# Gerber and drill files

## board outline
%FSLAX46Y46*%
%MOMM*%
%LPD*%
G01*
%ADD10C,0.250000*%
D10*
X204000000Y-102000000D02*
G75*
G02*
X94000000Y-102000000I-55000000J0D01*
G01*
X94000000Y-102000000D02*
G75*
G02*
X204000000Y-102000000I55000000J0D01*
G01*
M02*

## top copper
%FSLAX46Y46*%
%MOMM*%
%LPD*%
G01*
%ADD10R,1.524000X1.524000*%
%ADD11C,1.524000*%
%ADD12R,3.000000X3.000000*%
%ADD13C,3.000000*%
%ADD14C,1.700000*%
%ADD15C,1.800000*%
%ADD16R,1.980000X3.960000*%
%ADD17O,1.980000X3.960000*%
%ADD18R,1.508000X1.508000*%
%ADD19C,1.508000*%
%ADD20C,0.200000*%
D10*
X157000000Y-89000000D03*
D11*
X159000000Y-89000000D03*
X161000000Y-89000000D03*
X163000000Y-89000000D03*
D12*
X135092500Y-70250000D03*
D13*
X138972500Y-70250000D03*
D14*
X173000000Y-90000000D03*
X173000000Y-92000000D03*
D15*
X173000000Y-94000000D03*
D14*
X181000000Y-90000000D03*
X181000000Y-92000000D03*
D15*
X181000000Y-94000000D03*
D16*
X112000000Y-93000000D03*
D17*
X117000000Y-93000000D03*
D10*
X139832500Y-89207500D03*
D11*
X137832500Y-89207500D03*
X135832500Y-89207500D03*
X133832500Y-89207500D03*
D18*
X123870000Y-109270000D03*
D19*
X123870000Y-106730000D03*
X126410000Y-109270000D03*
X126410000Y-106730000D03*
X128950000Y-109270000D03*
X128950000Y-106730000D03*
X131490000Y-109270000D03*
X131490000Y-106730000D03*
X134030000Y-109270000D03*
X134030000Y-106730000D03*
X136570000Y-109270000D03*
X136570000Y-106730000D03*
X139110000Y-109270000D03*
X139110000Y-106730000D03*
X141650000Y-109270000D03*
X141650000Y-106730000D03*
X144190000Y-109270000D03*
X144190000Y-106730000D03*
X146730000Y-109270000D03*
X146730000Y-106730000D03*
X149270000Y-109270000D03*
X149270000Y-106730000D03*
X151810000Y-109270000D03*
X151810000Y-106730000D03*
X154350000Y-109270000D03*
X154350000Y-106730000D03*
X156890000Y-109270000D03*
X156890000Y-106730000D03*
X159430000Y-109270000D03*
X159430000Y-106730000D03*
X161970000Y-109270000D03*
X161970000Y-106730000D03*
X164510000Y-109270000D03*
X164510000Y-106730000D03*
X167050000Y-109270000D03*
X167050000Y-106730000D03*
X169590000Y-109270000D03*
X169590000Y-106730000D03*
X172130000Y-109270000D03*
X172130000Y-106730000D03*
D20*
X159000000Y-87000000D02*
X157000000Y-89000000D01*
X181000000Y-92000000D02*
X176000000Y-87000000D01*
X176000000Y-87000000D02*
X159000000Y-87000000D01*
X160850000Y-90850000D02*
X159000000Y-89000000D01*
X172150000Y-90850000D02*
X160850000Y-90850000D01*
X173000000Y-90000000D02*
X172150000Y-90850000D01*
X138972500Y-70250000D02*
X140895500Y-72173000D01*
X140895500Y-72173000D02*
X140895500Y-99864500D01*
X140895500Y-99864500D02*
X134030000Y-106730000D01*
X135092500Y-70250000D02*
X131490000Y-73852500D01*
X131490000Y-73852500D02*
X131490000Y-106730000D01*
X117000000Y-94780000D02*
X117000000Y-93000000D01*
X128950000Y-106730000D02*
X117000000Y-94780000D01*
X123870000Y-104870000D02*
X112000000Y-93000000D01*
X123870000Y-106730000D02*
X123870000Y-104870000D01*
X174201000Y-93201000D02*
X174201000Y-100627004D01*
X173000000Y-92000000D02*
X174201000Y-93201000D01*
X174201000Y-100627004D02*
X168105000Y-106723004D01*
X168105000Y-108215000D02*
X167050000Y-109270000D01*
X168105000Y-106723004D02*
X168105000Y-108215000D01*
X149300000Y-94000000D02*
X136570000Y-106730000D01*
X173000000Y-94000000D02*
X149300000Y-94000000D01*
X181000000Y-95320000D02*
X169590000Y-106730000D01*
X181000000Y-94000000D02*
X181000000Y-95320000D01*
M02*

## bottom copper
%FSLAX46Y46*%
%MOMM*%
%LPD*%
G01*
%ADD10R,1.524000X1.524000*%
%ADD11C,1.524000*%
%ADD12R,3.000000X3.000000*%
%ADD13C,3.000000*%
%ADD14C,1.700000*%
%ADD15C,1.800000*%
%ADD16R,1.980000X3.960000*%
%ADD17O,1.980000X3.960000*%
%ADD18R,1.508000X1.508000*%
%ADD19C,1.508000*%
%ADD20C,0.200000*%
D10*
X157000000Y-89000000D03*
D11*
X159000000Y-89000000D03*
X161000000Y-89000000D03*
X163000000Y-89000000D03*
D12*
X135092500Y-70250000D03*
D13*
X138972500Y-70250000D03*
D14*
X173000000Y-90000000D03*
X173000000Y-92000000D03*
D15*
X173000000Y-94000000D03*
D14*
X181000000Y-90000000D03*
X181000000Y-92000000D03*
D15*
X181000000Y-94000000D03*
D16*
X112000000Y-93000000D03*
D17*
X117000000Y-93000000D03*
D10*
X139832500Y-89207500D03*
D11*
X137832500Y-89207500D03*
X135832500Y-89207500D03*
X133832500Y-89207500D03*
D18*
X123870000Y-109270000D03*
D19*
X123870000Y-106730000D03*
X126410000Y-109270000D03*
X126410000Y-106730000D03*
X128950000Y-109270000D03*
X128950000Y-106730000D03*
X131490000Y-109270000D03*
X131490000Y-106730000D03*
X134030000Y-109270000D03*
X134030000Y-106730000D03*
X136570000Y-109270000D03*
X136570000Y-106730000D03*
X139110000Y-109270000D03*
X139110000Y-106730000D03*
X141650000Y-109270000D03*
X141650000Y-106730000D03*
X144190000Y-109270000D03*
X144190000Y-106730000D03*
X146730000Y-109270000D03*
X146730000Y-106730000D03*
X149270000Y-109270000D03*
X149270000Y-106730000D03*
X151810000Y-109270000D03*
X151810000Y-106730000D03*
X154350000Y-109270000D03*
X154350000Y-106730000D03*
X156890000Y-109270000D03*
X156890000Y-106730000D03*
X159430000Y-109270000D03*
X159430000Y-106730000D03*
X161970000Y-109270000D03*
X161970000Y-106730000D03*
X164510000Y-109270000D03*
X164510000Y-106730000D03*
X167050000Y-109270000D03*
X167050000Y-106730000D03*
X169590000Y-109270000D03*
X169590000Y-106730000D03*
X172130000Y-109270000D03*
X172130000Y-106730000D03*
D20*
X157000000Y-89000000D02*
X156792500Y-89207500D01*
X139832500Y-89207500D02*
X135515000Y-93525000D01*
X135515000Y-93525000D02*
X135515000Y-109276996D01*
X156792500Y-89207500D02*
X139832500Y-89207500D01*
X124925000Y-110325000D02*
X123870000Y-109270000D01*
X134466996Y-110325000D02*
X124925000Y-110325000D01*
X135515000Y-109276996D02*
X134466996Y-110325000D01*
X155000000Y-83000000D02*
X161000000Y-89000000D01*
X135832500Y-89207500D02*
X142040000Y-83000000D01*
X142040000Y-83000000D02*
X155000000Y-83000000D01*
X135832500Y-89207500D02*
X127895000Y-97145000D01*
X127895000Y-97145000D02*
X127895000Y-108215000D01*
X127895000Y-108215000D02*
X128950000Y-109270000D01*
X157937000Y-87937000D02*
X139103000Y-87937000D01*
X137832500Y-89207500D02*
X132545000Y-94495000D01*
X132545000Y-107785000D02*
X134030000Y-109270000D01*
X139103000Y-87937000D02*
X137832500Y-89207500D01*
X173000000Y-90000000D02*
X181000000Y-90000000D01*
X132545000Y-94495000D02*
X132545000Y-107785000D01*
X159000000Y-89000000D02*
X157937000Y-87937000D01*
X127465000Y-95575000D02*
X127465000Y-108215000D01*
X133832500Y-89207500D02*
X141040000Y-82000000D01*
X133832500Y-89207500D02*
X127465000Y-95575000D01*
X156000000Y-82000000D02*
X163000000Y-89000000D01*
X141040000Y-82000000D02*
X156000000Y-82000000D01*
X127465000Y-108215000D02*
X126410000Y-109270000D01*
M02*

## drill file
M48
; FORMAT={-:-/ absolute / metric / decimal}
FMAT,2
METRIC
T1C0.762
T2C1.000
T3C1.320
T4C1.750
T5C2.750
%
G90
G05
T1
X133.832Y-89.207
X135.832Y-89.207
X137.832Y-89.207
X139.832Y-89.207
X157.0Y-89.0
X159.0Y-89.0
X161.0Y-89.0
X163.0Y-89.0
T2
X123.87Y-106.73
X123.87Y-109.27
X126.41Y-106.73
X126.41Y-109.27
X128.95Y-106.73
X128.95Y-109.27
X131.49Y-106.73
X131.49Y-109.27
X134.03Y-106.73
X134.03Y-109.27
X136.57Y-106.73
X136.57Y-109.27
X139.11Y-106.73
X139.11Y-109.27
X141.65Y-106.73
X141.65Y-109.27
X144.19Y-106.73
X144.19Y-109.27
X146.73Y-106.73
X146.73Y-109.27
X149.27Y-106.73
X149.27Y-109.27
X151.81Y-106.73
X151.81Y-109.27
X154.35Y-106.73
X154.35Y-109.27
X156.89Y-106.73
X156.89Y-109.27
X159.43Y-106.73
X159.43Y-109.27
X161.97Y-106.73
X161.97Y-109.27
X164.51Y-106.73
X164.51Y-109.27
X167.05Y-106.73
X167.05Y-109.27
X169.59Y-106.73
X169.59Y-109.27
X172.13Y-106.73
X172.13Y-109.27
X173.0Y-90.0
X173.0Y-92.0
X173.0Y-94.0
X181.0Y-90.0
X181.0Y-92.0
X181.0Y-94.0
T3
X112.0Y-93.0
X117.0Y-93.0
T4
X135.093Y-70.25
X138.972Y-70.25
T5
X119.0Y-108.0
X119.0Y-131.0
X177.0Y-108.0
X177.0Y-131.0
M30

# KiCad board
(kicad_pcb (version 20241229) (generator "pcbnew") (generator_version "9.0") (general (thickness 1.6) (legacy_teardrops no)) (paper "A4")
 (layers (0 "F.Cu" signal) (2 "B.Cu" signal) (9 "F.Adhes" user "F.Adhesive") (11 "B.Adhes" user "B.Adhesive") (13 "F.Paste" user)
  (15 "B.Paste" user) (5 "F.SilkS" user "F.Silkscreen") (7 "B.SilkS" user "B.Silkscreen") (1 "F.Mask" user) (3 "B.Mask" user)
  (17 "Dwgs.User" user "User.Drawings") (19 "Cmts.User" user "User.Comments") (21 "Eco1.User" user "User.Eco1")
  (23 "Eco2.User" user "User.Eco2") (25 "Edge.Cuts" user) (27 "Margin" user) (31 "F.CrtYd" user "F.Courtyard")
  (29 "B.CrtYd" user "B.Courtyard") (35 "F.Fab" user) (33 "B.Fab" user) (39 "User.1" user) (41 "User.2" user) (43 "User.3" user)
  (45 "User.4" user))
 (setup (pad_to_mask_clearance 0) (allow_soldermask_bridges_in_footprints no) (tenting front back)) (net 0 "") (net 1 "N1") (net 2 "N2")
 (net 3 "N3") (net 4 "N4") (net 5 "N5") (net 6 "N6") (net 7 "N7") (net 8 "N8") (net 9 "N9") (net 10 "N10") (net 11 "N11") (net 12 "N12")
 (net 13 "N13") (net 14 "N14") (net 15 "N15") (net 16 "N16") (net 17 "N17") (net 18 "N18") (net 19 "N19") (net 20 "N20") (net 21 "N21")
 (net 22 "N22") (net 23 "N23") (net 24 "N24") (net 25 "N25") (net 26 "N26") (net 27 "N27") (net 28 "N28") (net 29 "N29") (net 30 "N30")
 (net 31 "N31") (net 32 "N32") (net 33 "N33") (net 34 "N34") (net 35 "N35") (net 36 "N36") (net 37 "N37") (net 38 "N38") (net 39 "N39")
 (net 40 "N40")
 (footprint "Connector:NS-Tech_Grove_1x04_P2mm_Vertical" (layer "F.Cu") (at 157 89 90)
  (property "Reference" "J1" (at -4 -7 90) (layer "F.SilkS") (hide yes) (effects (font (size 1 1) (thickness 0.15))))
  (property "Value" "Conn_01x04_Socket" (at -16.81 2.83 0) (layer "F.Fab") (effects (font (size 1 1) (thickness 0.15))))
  (pad "1" thru_hole rect (at 0 0 90) (size 1.524 1.524) (drill 0.762) (layers "*.Cu" "*.Mask") (remove_unused_layers no) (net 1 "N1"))
  (pad "2" thru_hole circle (at 0 2 90) (size 1.524 1.524) (drill 0.762) (layers "*.Cu" "*.Mask") (remove_unused_layers no) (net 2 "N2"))
  (pad "3" thru_hole circle (at 0 4 90) (size 1.524 1.524) (drill 0.762) (layers "*.Cu" "*.Mask") (remove_unused_layers no) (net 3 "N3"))
  (pad "4" thru_hole circle (at 0 6 90) (size 1.524 1.524) (drill 0.762) (layers "*.Cu" "*.Mask") (remove_unused_layers no) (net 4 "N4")))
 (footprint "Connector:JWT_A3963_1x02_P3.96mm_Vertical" (layer "F.Cu") (at 135.0925 70.25)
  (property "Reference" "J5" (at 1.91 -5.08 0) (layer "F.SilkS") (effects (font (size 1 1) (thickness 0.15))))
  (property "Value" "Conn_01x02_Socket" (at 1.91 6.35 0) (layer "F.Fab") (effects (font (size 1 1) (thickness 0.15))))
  (pad "1" thru_hole rect (at 0 0) (size 3 3) (drill 1.75) (layers "*.Cu" "*.Mask") (remove_unused_layers no) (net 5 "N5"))
  (pad "2" thru_hole circle (at 3.88 0) (size 3 3) (drill 1.75) (layers "*.Cu" "*.Mask") (remove_unused_layers no) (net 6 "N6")))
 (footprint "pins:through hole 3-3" (layer "F.Cu") (at 162 77)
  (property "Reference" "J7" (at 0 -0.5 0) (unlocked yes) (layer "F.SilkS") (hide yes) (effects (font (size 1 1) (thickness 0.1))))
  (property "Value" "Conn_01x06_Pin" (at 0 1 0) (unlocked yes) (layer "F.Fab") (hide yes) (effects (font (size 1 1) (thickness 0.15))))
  (pad "1" thru_hole circle (at 11 13) (size 1.7 1.7) (drill 1) (layers "*.Cu" "*.Mask") (remove_unused_layers no) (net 2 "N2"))
  (pad "2" thru_hole circle (at 11 15) (size 1.7 1.7) (drill 1) (layers "*.Cu" "*.Mask" "B.SilkS") (remove_unused_layers no) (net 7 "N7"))
  (pad "3" thru_hole circle (at 11 17) (size 1.8 1.8) (drill 1) (layers "*.Cu" "*.Mask") (remove_unused_layers no) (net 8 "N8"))
  (pad "4" thru_hole circle (at 19 13) (size 1.7 1.7) (drill 1) (layers "*.Cu" "*.Mask") (remove_unused_layers no) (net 2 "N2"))
  (pad "5" thru_hole circle (at 19 15) (size 1.7 1.7) (drill 1) (layers "*.Cu" "B.Mask" "B.Paste") (remove_unused_layers no) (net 1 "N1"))
  (pad "6" thru_hole circle (at 19 17) (size 1.8 1.8) (drill 1) (layers "*.Cu" "*.Mask") (remove_unused_layers no) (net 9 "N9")))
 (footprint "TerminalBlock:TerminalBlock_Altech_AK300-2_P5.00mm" (layer "F.Cu") (at 112 93)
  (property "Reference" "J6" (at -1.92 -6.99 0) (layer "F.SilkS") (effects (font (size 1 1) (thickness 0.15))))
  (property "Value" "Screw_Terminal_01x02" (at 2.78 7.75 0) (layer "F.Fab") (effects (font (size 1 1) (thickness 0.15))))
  (pad "1" thru_hole rect (at 0 0) (size 1.98 3.96) (drill 1.32) (layers "*.Cu" "*.Mask") (remove_unused_layers no) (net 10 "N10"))
  (pad "2" thru_hole oval (at 5 0) (size 1.98 3.96) (drill 1.32) (layers "*.Cu" "*.Mask") (remove_unused_layers no) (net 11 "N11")))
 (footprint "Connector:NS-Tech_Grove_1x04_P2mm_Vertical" (layer "F.Cu") (at 139.8325 89.2075 -90)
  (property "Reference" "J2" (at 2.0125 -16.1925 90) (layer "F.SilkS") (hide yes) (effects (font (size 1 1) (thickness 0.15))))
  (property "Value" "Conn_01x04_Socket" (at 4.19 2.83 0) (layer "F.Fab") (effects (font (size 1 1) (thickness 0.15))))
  (pad "1" thru_hole rect (at 0 0 270) (size 1.524 1.524) (drill 0.762) (layers "*.Cu" "*.Mask") (remove_unused_layers no) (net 1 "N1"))
  (pad "2" thru_hole circle (at 0 2 270) (size 1.524 1.524) (drill 0.762) (layers "*.Cu" "*.Mask") (remove_unused_layers no) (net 2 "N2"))
  (pad "3" thru_hole circle (at 0 4 270) (size 1.524 1.524) (drill 0.762) (layers "*.Cu" "*.Mask") (remove_unused_layers no) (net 3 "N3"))
  (pad "4" thru_hole circle (at 0 6 270) (size 1.524 1.524) (drill 0.762) (layers "*.Cu" "*.Mask") (remove_unused_layers no) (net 4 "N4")))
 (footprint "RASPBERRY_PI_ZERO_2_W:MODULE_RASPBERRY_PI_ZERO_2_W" (layer "F.Cu") (at 148 119.5)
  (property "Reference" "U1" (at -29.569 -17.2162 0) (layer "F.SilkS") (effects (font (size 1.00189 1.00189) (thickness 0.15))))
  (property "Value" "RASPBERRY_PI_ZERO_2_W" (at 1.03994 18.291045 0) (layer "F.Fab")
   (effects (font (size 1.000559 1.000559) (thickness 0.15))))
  (pad "" np_thru_hole circle (at -29 -11.5) (size 2.75 2.75) (drill 2.75) (layers "*.Cu" "*.Mask"))
  (pad "" np_thru_hole circle (at -29 11.5) (size 2.75 2.75) (drill 2.75) (layers "*.Cu" "*.Mask"))
  (pad "" np_thru_hole circle (at 29 -11.5) (size 2.75 2.75) (drill 2.75) (layers "*.Cu" "*.Mask"))
  (pad "" np_thru_hole circle (at 29 11.5) (size 2.75 2.75) (drill 2.75) (layers "*.Cu" "*.Mask"))
  (pad "1" thru_hole rect (at -24.13 -10.23) (size 1.508 1.508) (drill 1) (layers "*.Cu" "*.Mask") (remove_unused_layers no) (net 1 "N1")
   (solder_mask_margin 0.102))
  (pad "2" thru_hole circle (at -24.13 -12.77) (size 1.508 1.508) (drill 1) (layers "*.Cu" "*.Mask") (remove_unused_layers no)
   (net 10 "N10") (solder_mask_margin 0.102))
  (pad "3" thru_hole circle (at -21.59 -10.23) (size 1.508 1.508) (drill 1) (layers "*.Cu" "*.Mask") (remove_unused_layers no) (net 4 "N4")
   (solder_mask_margin 0.102))
  (pad "4" thru_hole circle (at -21.59 -12.77) (size 1.508 1.508) (drill 1) (layers "*.Cu" "*.Mask") (remove_unused_layers no)
   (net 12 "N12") (solder_mask_margin 0.102))
  (pad "5" thru_hole circle (at -19.05 -10.23) (size 1.508 1.508) (drill 1) (layers "*.Cu" "*.Mask") (remove_unused_layers no) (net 3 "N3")
   (solder_mask_margin 0.102))
  (pad "6" thru_hole circle (at -19.05 -12.77) (size 1.508 1.508) (drill 1) (layers "*.Cu" "*.Mask") (remove_unused_layers no)
   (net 11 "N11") (solder_mask_margin 0.102))
  (pad "7" thru_hole circle (at -16.51 -10.23) (size 1.508 1.508) (drill 1) (layers "*.Cu" "*.Mask") (remove_unused_layers no)
   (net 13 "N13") (solder_mask_margin 0.102))
  (pad "8" thru_hole circle (at -16.51 -12.77) (size 1.508 1.508) (drill 1) (layers "*.Cu" "*.Mask") (remove_unused_layers no) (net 5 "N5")
   (solder_mask_margin 0.102))
  (pad "9" thru_hole circle (at -13.97 -10.23) (size 1.508 1.508) (drill 1) (layers "*.Cu" "*.Mask") (remove_unused_layers no) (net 2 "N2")
   (solder_mask_margin 0.102))
  (pad "10" thru_hole circle (at -13.97 -12.77) (size 1.508 1.508) (drill 1) (layers "*.Cu" "*.Mask") (remove_unused_layers no) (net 6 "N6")
   (solder_mask_margin 0.102))
  (pad "11" thru_hole circle (at -11.43 -10.23) (size 1.508 1.508) (drill 1) (layers "*.Cu" "*.Mask") (remove_unused_layers no)
   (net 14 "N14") (solder_mask_margin 0.102))
  (pad "12" thru_hole circle (at -11.43 -12.77) (size 1.508 1.508) (drill 1) (layers "*.Cu" "*.Mask") (remove_unused_layers no) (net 8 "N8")
   (solder_mask_margin 0.102))
  (pad "13" thru_hole circle (at -8.89 -10.23) (size 1.508 1.508) (drill 1) (layers "*.Cu" "*.Mask") (remove_unused_layers no)
   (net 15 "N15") (solder_mask_margin 0.102))
  (pad "14" thru_hole circle (at -8.89 -12.77) (size 1.508 1.508) (drill 1) (layers "*.Cu" "*.Mask") (remove_unused_layers no)
   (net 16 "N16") (solder_mask_margin 0.102))
  (pad "15" thru_hole circle (at -6.35 -10.23) (size 1.508 1.508) (drill 1) (layers "*.Cu" "*.Mask") (remove_unused_layers no)
   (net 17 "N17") (solder_mask_margin 0.102))
  (pad "16" thru_hole circle (at -6.35 -12.77) (size 1.508 1.508) (drill 1) (layers "*.Cu" "*.Mask") (remove_unused_layers no)
   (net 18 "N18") (solder_mask_margin 0.102))
  (pad "17" thru_hole circle (at -3.81 -10.23) (size 1.508 1.508) (drill 1) (layers "*.Cu" "*.Mask") (remove_unused_layers no)
   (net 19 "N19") (solder_mask_margin 0.102))
  (pad "18" thru_hole circle (at -3.81 -12.77) (size 1.508 1.508) (drill 1) (layers "*.Cu" "*.Mask") (remove_unused_layers no)
   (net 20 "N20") (solder_mask_margin 0.102))
  (pad "19" thru_hole circle (at -1.27 -10.23) (size 1.508 1.508) (drill 1) (layers "*.Cu" "*.Mask") (remove_unused_layers no)
   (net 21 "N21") (solder_mask_margin 0.102))
  (pad "20" thru_hole circle (at -1.27 -12.77) (size 1.508 1.508) (drill 1) (layers "*.Cu" "*.Mask") (remove_unused_layers no)
   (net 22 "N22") (solder_mask_margin 0.102))
  (pad "21" thru_hole circle (at 1.27 -10.23) (size 1.508 1.508) (drill 1) (layers "*.Cu" "*.Mask") (remove_unused_layers no) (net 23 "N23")
   (solder_mask_margin 0.102))
  (pad "22" thru_hole circle (at 1.27 -12.77) (size 1.508 1.508) (drill 1) (layers "*.Cu" "*.Mask") (remove_unused_layers no) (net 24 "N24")
   (solder_mask_margin 0.102))
  (pad "23" thru_hole circle (at 3.81 -10.23) (size 1.508 1.508) (drill 1) (layers "*.Cu" "*.Mask") (remove_unused_layers no) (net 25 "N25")
   (solder_mask_margin 0.102))
  (pad "24" thru_hole circle (at 3.81 -12.77) (size 1.508 1.508) (drill 1) (layers "*.Cu" "*.Mask") (remove_unused_layers no) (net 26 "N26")
   (solder_mask_margin 0.102))
  (pad "25" thru_hole circle (at 6.35 -10.23) (size 1.508 1.508) (drill 1) (layers "*.Cu" "*.Mask") (remove_unused_layers no) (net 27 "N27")
   (solder_mask_margin 0.102))
  (pad "26" thru_hole circle (at 6.35 -12.77) (size 1.508 1.508) (drill 1) (layers "*.Cu" "*.Mask") (remove_unused_layers no) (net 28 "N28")
   (solder_mask_margin 0.102))
  (pad "27" thru_hole circle (at 8.89 -10.23) (size 1.508 1.508) (drill 1) (layers "*.Cu" "*.Mask") (remove_unused_layers no) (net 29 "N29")
   (solder_mask_margin 0.102))
  (pad "28" thru_hole circle (at 8.89 -12.77) (size 1.508 1.508) (drill 1) (layers "*.Cu" "*.Mask") (remove_unused_layers no) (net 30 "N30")
   (solder_mask_margin 0.102))
  (pad "29" thru_hole circle (at 11.43 -10.23) (size 1.508 1.508) (drill 1) (layers "*.Cu" "*.Mask") (remove_unused_layers no)
   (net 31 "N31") (solder_mask_margin 0.102))
  (pad "30" thru_hole circle (at 11.43 -12.77) (size 1.508 1.508) (drill 1) (layers "*.Cu" "*.Mask") (remove_unused_layers no)
   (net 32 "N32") (solder_mask_margin 0.102))
  (pad "31" thru_hole circle (at 13.97 -10.23) (size 1.508 1.508) (drill 1) (layers "*.Cu" "*.Mask") (remove_unused_layers no)
   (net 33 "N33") (solder_mask_margin 0.102))
  (pad "32" thru_hole circle (at 13.97 -12.77) (size 1.508 1.508) (drill 1) (layers "*.Cu" "*.Mask") (remove_unused_layers no)
   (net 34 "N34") (solder_mask_margin 0.102))
  (pad "33" thru_hole circle (at 16.51 -10.23) (size 1.508 1.508) (drill 1) (layers "*.Cu" "*.Mask") (remove_unused_layers no)
   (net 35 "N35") (solder_mask_margin 0.102))
  (pad "34" thru_hole circle (at 16.51 -12.77) (size 1.508 1.508) (drill 1) (layers "*.Cu" "*.Mask") (remove_unused_layers no)
   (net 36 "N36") (solder_mask_margin 0.102))
  (pad "35" thru_hole circle (at 19.05 -10.23) (size 1.508 1.508) (drill 1) (layers "*.Cu" "*.Mask") (remove_unused_layers no) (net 7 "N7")
   (solder_mask_margin 0.102))
  (pad "36" thru_hole circle (at 19.05 -12.77) (size 1.508 1.508) (drill 1) (layers "*.Cu" "*.Mask") (remove_unused_layers no)
   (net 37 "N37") (solder_mask_margin 0.102))
  (pad "37" thru_hole circle (at 21.59 -10.23) (size 1.508 1.508) (drill 1) (layers "*.Cu" "*.Mask") (remove_unused_layers no)
   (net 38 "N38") (solder_mask_margin 0.102))
  (pad "38" thru_hole circle (at 21.59 -12.77) (size 1.508 1.508) (drill 1) (layers "*.Cu" "*.Mask") (remove_unused_layers no) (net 9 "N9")
   (solder_mask_margin 0.102))
  (pad "39" thru_hole circle (at 24.13 -10.23) (size 1.508 1.508) (drill 1) (layers "*.Cu" "*.Mask") (remove_unused_layers no)
   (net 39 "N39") (solder_mask_margin 0.102))
  (pad "40" thru_hole circle (at 24.13 -12.77) (size 1.508 1.508) (drill 1) (layers "*.Cu" "*.Mask") (remove_unused_layers no)
   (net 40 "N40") (solder_mask_margin 0.102)))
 (gr_circle (center 149 102) (end 204 102) (stroke (width 0.25) (type solid)) (fill no) (layer "Edge.Cuts"))
 (segment (start 159 87) (end 157 89) (width 0.2) (layer "F.Cu") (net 1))
 (segment (start 181 92) (end 176 87) (width 0.2) (layer "F.Cu") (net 1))
 (segment (start 176 87) (end 159 87) (width 0.2) (layer "F.Cu") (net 1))
 (segment (start 157 89) (end 156.7925 89.2075) (width 0.2) (layer "B.Cu") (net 1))
 (segment (start 139.8325 89.2075) (end 135.515 93.525) (width 0.2) (layer "B.Cu") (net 1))
 (segment (start 135.515 93.525) (end 135.515 109.276996) (width 0.2) (layer "B.Cu") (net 1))
 (segment (start 156.7925 89.2075) (end 139.8325 89.2075) (width 0.2) (layer "B.Cu") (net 1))
 (segment (start 124.925 110.325) (end 123.87 109.27) (width 0.2) (layer "B.Cu") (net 1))
 (segment (start 134.466996 110.325) (end 124.925 110.325) (width 0.2) (layer "B.Cu") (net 1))
 (segment (start 135.515 109.276996) (end 134.466996 110.325) (width 0.2) (layer "B.Cu") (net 1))
 (segment (start 155 83) (end 161 89) (width 0.2) (layer "B.Cu") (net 3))
 (segment (start 135.8325 89.2075) (end 142.04 83) (width 0.2) (layer "B.Cu") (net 3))
 (segment (start 142.04 83) (end 155 83) (width 0.2) (layer "B.Cu") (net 3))
 (segment (start 135.8325 89.2075) (end 127.895 97.145) (width 0.2) (layer "B.Cu") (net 3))
 (segment (start 127.895 97.145) (end 127.895 108.215) (width 0.2) (layer "B.Cu") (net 3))
 (segment (start 127.895 108.215) (end 128.95 109.27) (width 0.2) (layer "B.Cu") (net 3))
 (segment (start 160.85 90.85) (end 159 89) (width 0.2) (layer "F.Cu") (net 2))
 (segment (start 172.15 90.85) (end 160.85 90.85) (width 0.2) (layer "F.Cu") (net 2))
 (segment (start 173 90) (end 172.15 90.85) (width 0.2) (layer "F.Cu") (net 2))
 (segment (start 157.937 87.937) (end 139.103 87.937) (width 0.2) (layer "B.Cu") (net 2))
 (segment (start 137.8325 89.2075) (end 132.545 94.495) (width 0.2) (layer "B.Cu") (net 2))
 (segment (start 132.545 107.785) (end 134.03 109.27) (width 0.2) (layer "B.Cu") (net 2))
 (segment (start 139.103 87.937) (end 137.8325 89.2075) (width 0.2) (layer "B.Cu") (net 2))
 (segment (start 173 90) (end 181 90) (width 0.2) (layer "B.Cu") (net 2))
 (segment (start 132.545 94.495) (end 132.545 107.785) (width 0.2) (layer "B.Cu") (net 2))
 (segment (start 159 89) (end 157.937 87.937) (width 0.2) (layer "B.Cu") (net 2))
 (segment (start 127.465 95.575) (end 127.465 108.215) (width 0.2) (layer "B.Cu") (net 4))
 (segment (start 133.8325 89.2075) (end 141.04 82) (width 0.2) (layer "B.Cu") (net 4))
 (segment (start 133.8325 89.2075) (end 127.465 95.575) (width 0.2) (layer "B.Cu") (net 4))
 (segment (start 156 82) (end 163 89) (width 0.2) (layer "B.Cu") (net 4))
 (segment (start 141.04 82) (end 156 82) (width 0.2) (layer "B.Cu") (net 4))
 (segment (start 127.465 108.215) (end 126.41 109.27) (width 0.2) (layer "B.Cu") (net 4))
 (segment (start 138.9725 70.25) (end 140.8955 72.173) (width 0.2) (layer "F.Cu") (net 6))
 (segment (start 140.8955 72.173) (end 140.8955 99.8645) (width 0.2) (layer "F.Cu") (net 6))
 (segment (start 140.8955 99.8645) (end 134.03 106.73) (width 0.2) (layer "F.Cu") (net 6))
 (segment (start 135.0925 70.25) (end 131.49 73.8525) (width 0.2) (layer "F.Cu") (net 5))
 (segment (start 131.49 73.8525) (end 131.49 106.73) (width 0.2) (layer "F.Cu") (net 5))
 (segment (start 117 94.78) (end 117 93) (width 0.2) (layer "F.Cu") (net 11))
 (segment (start 128.95 106.73) (end 117 94.78) (width 0.2) (layer "F.Cu") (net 11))
 (segment (start 123.87 104.87) (end 112 93) (width 0.2) (layer "F.Cu") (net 10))
 (segment (start 123.87 106.73) (end 123.87 104.87) (width 0.2) (layer "F.Cu") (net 10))
 (segment (start 174.201 93.201) (end 174.201 100.627004) (width 0.2) (layer "F.Cu") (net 7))
 (segment (start 173 92) (end 174.201 93.201) (width 0.2) (layer "F.Cu") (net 7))
 (segment (start 174.201 100.627004) (end 168.105 106.723004) (width 0.2) (layer "F.Cu") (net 7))
 (segment (start 168.105 108.215) (end 167.05 109.27) (width 0.2) (layer "F.Cu") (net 7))
 (segment (start 168.105 106.723004) (end 168.105 108.215) (width 0.2) (layer "F.Cu") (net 7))
 (segment (start 149.3 94) (end 136.57 106.73) (width 0.2) (layer "F.Cu") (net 8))
 (segment (start 173 94) (end 149.3 94) (width 0.2) (layer "F.Cu") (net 8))
 (segment (start 181 95.32) (end 169.59 106.73) (width 0.2) (layer "F.Cu") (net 9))
 (segment (start 181 94) (end 181 95.32) (width 0.2) (layer "F.Cu") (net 9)))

